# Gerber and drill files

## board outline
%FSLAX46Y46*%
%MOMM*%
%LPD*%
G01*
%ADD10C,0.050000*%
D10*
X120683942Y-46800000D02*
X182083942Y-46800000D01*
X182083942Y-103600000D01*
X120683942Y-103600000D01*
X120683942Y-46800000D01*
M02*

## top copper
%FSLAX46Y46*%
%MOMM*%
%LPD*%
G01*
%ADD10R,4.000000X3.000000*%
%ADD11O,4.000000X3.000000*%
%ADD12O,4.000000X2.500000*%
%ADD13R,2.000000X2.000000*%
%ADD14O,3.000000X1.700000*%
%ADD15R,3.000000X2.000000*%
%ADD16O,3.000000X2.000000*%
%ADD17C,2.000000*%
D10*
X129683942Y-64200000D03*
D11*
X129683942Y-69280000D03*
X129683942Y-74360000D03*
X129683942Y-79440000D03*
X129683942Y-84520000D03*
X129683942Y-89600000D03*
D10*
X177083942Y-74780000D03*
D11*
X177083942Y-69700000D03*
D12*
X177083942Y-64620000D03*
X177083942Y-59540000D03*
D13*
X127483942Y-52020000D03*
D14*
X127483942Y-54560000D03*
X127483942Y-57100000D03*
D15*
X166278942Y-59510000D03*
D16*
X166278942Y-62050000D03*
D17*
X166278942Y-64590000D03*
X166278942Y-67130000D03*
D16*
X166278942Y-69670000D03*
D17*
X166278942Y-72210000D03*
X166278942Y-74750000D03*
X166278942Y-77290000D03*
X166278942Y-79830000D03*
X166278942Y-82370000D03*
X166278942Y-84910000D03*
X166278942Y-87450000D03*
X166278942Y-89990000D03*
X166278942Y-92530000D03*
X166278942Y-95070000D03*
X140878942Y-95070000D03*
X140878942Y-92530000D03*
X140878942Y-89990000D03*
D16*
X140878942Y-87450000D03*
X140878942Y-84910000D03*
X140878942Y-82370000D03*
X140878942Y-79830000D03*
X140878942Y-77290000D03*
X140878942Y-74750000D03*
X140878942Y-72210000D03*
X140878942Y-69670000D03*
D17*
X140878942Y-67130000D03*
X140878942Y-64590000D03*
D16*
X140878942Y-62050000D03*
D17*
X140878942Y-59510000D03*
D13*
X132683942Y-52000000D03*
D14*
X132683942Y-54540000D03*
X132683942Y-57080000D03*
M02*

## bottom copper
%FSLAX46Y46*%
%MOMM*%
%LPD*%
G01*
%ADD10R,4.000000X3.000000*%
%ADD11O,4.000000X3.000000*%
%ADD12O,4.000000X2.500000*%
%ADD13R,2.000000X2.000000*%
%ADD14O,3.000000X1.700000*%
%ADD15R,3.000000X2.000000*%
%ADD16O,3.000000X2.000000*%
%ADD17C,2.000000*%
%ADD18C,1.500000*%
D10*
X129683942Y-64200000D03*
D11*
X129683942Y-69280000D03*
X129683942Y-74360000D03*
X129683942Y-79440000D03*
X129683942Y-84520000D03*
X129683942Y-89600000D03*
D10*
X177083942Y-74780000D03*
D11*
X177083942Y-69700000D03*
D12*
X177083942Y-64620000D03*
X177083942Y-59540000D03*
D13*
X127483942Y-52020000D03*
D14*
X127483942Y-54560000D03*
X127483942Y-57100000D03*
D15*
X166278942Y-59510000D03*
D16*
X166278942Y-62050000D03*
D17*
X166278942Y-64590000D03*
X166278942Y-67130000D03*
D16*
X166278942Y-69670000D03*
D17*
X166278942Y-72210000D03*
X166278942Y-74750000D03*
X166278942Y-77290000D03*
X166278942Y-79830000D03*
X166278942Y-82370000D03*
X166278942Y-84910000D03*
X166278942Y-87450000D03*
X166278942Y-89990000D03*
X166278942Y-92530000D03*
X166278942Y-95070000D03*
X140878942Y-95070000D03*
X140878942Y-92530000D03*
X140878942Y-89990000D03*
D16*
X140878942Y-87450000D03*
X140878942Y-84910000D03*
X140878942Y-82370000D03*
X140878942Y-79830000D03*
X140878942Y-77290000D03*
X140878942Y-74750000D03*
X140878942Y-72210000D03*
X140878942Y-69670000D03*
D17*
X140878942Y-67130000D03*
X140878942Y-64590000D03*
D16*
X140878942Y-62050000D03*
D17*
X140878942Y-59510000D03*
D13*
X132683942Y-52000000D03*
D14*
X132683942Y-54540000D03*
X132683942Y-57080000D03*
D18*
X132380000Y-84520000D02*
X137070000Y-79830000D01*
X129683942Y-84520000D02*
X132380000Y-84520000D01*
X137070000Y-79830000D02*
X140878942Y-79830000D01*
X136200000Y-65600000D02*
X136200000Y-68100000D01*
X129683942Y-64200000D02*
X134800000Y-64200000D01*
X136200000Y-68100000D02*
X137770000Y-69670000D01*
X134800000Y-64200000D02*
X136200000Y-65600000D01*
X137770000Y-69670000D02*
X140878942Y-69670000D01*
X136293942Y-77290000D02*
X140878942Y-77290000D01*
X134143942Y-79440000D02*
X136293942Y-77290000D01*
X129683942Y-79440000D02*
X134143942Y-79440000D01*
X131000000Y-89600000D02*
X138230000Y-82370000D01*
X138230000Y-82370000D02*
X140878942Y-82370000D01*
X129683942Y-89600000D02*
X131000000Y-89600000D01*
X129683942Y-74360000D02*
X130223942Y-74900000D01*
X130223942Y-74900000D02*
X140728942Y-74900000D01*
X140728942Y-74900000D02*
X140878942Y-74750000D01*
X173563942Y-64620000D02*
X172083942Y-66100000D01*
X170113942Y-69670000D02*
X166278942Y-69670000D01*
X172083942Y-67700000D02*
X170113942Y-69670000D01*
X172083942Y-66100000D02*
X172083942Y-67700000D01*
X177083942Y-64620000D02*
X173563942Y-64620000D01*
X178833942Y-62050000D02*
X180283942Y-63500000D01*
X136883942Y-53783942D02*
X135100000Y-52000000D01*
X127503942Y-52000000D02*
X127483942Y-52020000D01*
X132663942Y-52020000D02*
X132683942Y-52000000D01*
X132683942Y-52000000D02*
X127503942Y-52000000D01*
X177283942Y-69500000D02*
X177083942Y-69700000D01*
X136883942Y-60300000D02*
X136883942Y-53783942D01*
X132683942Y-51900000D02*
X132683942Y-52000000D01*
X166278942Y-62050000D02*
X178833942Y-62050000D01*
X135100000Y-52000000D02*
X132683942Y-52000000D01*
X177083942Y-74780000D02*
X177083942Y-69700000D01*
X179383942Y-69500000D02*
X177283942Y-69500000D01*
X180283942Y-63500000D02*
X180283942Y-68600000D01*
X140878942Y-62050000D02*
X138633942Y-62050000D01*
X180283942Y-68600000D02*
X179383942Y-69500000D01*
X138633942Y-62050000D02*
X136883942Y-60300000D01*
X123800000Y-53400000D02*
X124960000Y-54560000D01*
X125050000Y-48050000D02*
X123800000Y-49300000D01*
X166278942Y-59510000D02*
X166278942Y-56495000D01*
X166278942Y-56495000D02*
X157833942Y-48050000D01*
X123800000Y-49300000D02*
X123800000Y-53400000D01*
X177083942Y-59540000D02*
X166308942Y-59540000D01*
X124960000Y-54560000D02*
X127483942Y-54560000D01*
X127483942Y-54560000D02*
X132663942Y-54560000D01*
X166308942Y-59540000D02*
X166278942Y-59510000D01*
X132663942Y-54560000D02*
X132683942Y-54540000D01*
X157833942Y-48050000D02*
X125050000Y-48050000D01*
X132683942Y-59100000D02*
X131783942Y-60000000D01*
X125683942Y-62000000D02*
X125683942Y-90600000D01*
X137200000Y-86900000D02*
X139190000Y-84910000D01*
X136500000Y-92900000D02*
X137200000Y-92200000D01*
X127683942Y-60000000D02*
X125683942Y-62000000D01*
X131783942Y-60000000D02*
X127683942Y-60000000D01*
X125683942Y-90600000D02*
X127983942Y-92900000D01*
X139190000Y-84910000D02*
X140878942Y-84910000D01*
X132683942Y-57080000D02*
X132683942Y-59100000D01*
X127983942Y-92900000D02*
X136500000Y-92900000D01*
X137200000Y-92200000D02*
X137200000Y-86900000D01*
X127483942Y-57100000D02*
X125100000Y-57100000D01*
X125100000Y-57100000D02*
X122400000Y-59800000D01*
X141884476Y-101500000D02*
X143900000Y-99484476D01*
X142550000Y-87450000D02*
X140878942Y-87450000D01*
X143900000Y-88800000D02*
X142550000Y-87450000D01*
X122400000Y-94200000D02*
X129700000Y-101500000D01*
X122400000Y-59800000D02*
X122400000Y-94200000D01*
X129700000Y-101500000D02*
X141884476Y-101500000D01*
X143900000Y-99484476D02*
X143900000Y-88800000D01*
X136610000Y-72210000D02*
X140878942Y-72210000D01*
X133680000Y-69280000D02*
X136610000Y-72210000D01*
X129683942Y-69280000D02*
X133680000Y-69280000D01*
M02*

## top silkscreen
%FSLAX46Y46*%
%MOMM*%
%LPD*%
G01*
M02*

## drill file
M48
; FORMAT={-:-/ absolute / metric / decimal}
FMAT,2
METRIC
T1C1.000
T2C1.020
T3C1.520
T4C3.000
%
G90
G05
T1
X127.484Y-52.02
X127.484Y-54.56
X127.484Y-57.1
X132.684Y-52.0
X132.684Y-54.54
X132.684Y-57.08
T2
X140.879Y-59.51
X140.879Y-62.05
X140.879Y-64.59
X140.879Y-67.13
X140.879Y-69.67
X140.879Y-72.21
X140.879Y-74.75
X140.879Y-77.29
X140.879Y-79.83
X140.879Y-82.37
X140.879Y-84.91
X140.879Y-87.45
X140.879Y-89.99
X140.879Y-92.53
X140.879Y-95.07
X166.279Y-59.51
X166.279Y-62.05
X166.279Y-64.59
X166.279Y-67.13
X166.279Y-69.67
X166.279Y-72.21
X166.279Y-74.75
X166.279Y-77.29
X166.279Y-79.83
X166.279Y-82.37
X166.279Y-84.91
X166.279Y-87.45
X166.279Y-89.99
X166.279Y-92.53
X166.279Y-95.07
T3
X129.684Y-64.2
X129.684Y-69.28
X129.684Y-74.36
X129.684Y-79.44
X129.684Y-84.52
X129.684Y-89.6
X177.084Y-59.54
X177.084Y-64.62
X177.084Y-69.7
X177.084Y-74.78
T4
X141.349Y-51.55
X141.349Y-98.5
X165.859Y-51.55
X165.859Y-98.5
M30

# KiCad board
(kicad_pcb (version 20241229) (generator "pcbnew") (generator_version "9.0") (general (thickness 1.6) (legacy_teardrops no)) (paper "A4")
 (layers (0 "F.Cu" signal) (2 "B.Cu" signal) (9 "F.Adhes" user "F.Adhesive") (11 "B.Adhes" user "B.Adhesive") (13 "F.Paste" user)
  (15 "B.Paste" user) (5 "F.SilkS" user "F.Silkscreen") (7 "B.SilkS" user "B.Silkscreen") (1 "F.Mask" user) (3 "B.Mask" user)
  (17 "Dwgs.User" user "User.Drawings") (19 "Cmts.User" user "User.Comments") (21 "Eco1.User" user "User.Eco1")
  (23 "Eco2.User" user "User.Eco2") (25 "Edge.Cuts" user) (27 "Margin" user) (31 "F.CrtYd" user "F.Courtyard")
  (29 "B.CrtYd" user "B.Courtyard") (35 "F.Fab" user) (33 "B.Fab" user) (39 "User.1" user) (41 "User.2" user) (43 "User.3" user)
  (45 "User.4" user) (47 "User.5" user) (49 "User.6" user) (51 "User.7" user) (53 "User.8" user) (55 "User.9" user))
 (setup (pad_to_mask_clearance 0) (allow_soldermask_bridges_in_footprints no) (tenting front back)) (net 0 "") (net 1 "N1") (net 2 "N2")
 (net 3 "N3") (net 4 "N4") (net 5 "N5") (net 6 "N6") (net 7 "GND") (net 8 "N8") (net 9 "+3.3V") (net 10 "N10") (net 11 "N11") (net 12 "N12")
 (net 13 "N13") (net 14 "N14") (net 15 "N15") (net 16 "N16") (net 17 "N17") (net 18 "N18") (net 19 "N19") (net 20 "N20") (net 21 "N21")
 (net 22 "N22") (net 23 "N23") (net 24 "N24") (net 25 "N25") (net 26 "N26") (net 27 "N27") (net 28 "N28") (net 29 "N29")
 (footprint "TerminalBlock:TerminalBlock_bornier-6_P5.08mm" (layer "B.Cu") (at 129.683942 64.2 -90)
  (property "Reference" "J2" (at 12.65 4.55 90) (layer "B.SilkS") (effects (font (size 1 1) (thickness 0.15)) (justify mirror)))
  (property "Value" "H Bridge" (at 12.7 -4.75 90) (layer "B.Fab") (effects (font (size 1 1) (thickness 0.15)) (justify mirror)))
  (pad "1" thru_hole rect (at 0 0 270) (size 3 4) (drill 1.52) (layers "*.Cu" "*.Mask") (remove_unused_layers no) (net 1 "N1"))
  (pad "2" thru_hole oval (at 5.08 0 270) (size 3 4) (drill 1.52) (layers "*.Cu" "*.Mask") (remove_unused_layers no) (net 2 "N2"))
  (pad "3" thru_hole oval (at 10.16 0 270) (size 3 4) (drill 1.52) (layers "*.Cu" "*.Mask") (remove_unused_layers no) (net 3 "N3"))
  (pad "4" thru_hole oval (at 15.24 0 270) (size 3 4) (drill 1.52) (layers "*.Cu" "*.Mask") (remove_unused_layers no) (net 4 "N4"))
  (pad "5" thru_hole oval (at 20.32 0 270) (size 3 4) (drill 1.52) (layers "*.Cu" "*.Mask") (remove_unused_layers no) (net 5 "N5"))
  (pad "6" thru_hole oval (at 25.4 0 270) (size 3 4) (drill 1.52) (layers "*.Cu" "*.Mask") (remove_unused_layers no) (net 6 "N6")))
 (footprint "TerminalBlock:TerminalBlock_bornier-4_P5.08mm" (layer "B.Cu") (at 177.083942 74.78 90)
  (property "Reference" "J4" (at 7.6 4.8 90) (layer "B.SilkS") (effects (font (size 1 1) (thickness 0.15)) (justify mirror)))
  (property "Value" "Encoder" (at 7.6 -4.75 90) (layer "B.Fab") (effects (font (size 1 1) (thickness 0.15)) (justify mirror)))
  (pad "1" thru_hole rect (at 0 0 90) (size 3 4) (drill 1.52) (layers "*.Cu" "*.Mask") (remove_unused_layers no) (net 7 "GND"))
  (pad "2" thru_hole oval (at 5.08 0 90) (size 3 4) (drill 1.52) (layers "*.Cu" "*.Mask") (remove_unused_layers no) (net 7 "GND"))
  (pad "3" thru_hole oval (at 10.16 0 90) (size 2.5 4) (drill 1.52) (layers "*.Cu" "*.Mask") (remove_unused_layers no) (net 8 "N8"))
  (pad "4" thru_hole oval (at 15.24 0 90) (size 2.5 4) (drill 1.52) (layers "*.Cu" "*.Mask") (remove_unused_layers no) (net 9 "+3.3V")))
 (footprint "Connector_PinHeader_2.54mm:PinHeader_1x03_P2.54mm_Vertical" (layer "B.Cu") (at 127.483942 52.02 180)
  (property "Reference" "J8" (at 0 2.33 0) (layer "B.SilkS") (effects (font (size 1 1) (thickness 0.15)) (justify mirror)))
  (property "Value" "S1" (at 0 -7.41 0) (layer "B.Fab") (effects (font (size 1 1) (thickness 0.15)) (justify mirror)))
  (pad "1" thru_hole rect (at 0 0 180) (size 2 2) (drill 1) (layers "*.Cu" "*.Mask") (remove_unused_layers no) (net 7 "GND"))
  (pad "2" thru_hole oval (at 0 -2.54 180) (size 3 1.7) (drill 1) (layers "*.Cu" "*.Mask") (remove_unused_layers no) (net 9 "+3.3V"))
  (pad "3" thru_hole oval (at 0 -5.08 180) (size 3 1.7) (drill 1) (layers "*.Cu" "*.Mask") (remove_unused_layers no) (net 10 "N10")))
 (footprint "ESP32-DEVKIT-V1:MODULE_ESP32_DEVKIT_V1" (layer "B.Cu") (at 153.578942 75.025 180)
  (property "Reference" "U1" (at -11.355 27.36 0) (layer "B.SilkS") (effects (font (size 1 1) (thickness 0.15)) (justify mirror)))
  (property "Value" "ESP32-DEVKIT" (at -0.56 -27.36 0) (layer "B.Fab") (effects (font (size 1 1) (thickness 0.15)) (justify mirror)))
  (pad "" np_thru_hole circle (at -12.28 -23.475 180) (size 3 3) (drill 3) (layers "*.Cu" "*.Mask"))
  (pad "" np_thru_hole circle (at -12.28 23.475 180) (size 3 3) (drill 3) (layers "*.Cu" "*.Mask"))
  (pad "" np_thru_hole circle (at 12.23 -23.475 180) (size 3 3) (drill 3) (layers "*.Cu" "*.Mask"))
  (pad "" np_thru_hole circle (at 12.23 23.475 180) (size 3 3) (drill 3) (layers "*.Cu" "*.Mask"))
  (pad "1" thru_hole rect (at -12.7 15.515 180) (size 3 2) (drill 1.02) (layers "*.Cu" "*.Mask") (remove_unused_layers no) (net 9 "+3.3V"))
  (pad "2" thru_hole oval (at -12.7 12.975 180) (size 3 2) (drill 1.02) (layers "*.Cu" "*.Mask") (remove_unused_layers no) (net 7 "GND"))
  (pad "3" thru_hole circle (at -12.7 10.435 180) (size 2 2) (drill 1.02) (layers "*.Cu" "*.Mask") (remove_unused_layers no) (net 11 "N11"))
  (pad "4" thru_hole circle (at -12.7 7.895 180) (size 2 2) (drill 1.02) (layers "*.Cu" "*.Mask") (remove_unused_layers no) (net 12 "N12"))
  (pad "5" thru_hole oval (at -12.7 5.355 180) (size 3 2) (drill 1.02) (layers "*.Cu" "*.Mask") (remove_unused_layers no) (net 8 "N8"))
  (pad "6" thru_hole circle (at -12.7 2.815 180) (size 2 2) (drill 1.02) (layers "*.Cu" "*.Mask") (remove_unused_layers no) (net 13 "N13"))
  (pad "7" thru_hole circle (at -12.7 0.275 180) (size 2 2) (drill 1.02) (layers "*.Cu" "*.Mask") (remove_unused_layers no) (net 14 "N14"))
  (pad "8" thru_hole circle (at -12.7 -2.265 180) (size 2 2) (drill 1.02) (layers "*.Cu" "*.Mask") (remove_unused_layers no) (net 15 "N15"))
  (pad "9" thru_hole circle (at -12.7 -4.805 180) (size 2 2) (drill 1.02) (layers "*.Cu" "*.Mask") (remove_unused_layers no) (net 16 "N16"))
  (pad "10" thru_hole circle (at -12.7 -7.345 180) (size 2 2) (drill 1.02) (layers "*.Cu" "*.Mask") (remove_unused_layers no) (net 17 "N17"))
  (pad "11" thru_hole circle (at -12.7 -9.885 180) (size 2 2) (drill 1.02) (layers "*.Cu" "*.Mask") (remove_unused_layers no) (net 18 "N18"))
  (pad "12" thru_hole circle (at -12.7 -12.425 180) (size 2 2) (drill 1.02) (layers "*.Cu" "*.Mask") (remove_unused_layers no)
   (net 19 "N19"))
  (pad "13" thru_hole circle (at -12.7 -14.965 180) (size 2 2) (drill 1.02) (layers "*.Cu" "*.Mask") (remove_unused_layers no)
   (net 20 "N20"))
  (pad "14" thru_hole circle (at -12.7 -17.505 180) (size 2 2) (drill 1.02) (layers "*.Cu" "*.Mask") (remove_unused_layers no)
   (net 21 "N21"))
  (pad "15" thru_hole circle (at -12.7 -20.045 180) (size 2 2) (drill 1.02) (layers "*.Cu" "*.Mask") (remove_unused_layers no)
   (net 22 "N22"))
  (pad "16" thru_hole circle (at 12.7 -20.045 180) (size 2 2) (drill 1.02) (layers "*.Cu" "*.Mask") (remove_unused_layers no) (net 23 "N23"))
  (pad "17" thru_hole circle (at 12.7 -17.505 180) (size 2 2) (drill 1.02) (layers "*.Cu" "*.Mask") (remove_unused_layers no) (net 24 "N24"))
  (pad "18" thru_hole circle (at 12.7 -14.965 180) (size 2 2) (drill 1.02) (layers "*.Cu" "*.Mask") (remove_unused_layers no) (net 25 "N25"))
  (pad "19" thru_hole oval (at 12.7 -12.425 180) (size 3 2) (drill 1.02) (layers "*.Cu" "*.Mask") (remove_unused_layers no) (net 10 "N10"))
  (pad "20" thru_hole oval (at 12.7 -9.885 180) (size 3 2) (drill 1.02) (layers "*.Cu" "*.Mask") (remove_unused_layers no) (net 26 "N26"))
  (pad "21" thru_hole oval (at 12.7 -7.345 180) (size 3 2) (drill 1.02) (layers "*.Cu" "*.Mask") (remove_unused_layers no) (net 6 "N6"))
  (pad "22" thru_hole oval (at 12.7 -4.805 180) (size 3 2) (drill 1.02) (layers "*.Cu" "*.Mask") (remove_unused_layers no) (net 5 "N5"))
  (pad "23" thru_hole oval (at 12.7 -2.265 180) (size 3 2) (drill 1.02) (layers "*.Cu" "*.Mask") (remove_unused_layers no) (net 4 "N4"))
  (pad "24" thru_hole oval (at 12.7 0.275 180) (size 3 2) (drill 1.02) (layers "*.Cu" "*.Mask") (remove_unused_layers no) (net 3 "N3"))
  (pad "25" thru_hole oval (at 12.7 2.815 180) (size 3 2) (drill 1.02) (layers "*.Cu" "*.Mask") (remove_unused_layers no) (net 2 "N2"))
  (pad "26" thru_hole oval (at 12.7 5.355 180) (size 3 2) (drill 1.02) (layers "*.Cu" "*.Mask") (remove_unused_layers no) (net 1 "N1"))
  (pad "27" thru_hole circle (at 12.7 7.895 180) (size 2 2) (drill 1.02) (layers "*.Cu" "*.Mask") (remove_unused_layers no) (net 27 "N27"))
  (pad "28" thru_hole circle (at 12.7 10.435 180) (size 2 2) (drill 1.02) (layers "*.Cu" "*.Mask") (remove_unused_layers no) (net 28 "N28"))
  (pad "29" thru_hole oval (at 12.7 12.975 180) (size 3 2) (drill 1.02) (layers "*.Cu" "*.Mask") (remove_unused_layers no) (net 7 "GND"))
  (pad "30" thru_hole circle (at 12.7 15.515 180) (size 2 2) (drill 1.02) (layers "*.Cu" "*.Mask") (remove_unused_layers no) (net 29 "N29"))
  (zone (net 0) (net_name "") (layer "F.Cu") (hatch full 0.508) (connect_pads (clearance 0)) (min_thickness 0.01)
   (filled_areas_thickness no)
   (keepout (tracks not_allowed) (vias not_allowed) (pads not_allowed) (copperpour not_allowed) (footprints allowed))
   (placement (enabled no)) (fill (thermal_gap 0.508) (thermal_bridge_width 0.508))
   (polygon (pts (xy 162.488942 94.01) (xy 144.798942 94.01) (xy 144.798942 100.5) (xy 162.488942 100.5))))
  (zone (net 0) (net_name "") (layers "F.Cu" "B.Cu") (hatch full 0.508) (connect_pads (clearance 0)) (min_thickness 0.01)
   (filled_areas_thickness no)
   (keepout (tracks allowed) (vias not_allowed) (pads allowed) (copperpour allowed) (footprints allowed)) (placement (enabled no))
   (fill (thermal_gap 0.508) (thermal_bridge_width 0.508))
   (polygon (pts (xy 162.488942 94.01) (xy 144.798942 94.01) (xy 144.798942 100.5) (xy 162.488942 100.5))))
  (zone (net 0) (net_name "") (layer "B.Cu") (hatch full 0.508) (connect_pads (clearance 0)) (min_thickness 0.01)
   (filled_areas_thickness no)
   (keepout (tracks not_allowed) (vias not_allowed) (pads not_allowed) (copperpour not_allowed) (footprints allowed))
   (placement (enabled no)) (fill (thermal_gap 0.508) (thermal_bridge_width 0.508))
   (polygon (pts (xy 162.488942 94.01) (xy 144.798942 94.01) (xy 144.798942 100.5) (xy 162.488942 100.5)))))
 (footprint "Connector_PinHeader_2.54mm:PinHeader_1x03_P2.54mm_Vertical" (layer "B.Cu") (at 132.683942 52 180)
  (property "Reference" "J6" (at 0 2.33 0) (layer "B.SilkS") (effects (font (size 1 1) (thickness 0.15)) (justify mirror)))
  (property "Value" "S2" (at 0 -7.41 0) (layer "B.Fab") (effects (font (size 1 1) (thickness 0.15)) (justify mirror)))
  (pad "1" thru_hole rect (at 0 0 180) (size 2 2) (drill 1) (layers "*.Cu" "*.Mask") (remove_unused_layers no) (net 7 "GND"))
  (pad "2" thru_hole oval (at 0 -2.54 180) (size 3 1.7) (drill 1) (layers "*.Cu" "*.Mask") (remove_unused_layers no) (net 9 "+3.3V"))
  (pad "3" thru_hole oval (at 0 -5.08 180) (size 3 1.7) (drill 1) (layers "*.Cu" "*.Mask") (remove_unused_layers no) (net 26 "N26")))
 (gr_rect (start 120.683942 46.8) (end 182.083942 103.6) (stroke (width 0.05) (type default)) (fill no) (layer "Edge.Cuts"))
 (segment (start 132.38 84.52) (end 137.07 79.83) (width 1.5) (layer "B.Cu") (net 5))
 (segment (start 129.683942 84.52) (end 132.38 84.52) (width 1.5) (layer "B.Cu") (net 5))
 (segment (start 137.07 79.83) (end 140.878942 79.83) (width 1.5) (layer "B.Cu") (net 5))
 (segment (start 136.2 65.6) (end 136.2 68.1) (width 1.5) (layer "B.Cu") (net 1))
 (segment (start 129.683942 64.2) (end 134.8 64.2) (width 1.5) (layer "B.Cu") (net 1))
 (segment (start 136.2 68.1) (end 137.77 69.67) (width 1.5) (layer "B.Cu") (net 1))
 (segment (start 134.8 64.2) (end 136.2 65.6) (width 1.5) (layer "B.Cu") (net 1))
 (segment (start 137.77 69.67) (end 140.878942 69.67) (width 1.5) (layer "B.Cu") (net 1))
 (segment (start 136.293942 77.29) (end 140.878942 77.29) (width 1.5) (layer "B.Cu") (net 4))
 (segment (start 134.143942 79.44) (end 136.293942 77.29) (width 1.5) (layer "B.Cu") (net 4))
 (segment (start 129.683942 79.44) (end 134.143942 79.44) (width 1.5) (layer "B.Cu") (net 4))
 (segment (start 131 89.6) (end 138.23 82.37) (width 1.5) (layer "B.Cu") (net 6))
 (segment (start 138.23 82.37) (end 140.878942 82.37) (width 1.5) (layer "B.Cu") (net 6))
 (segment (start 129.683942 89.6) (end 131 89.6) (width 1.5) (layer "B.Cu") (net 6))
 (segment (start 129.683942 74.36) (end 130.223942 74.9) (width 1.5) (layer "B.Cu") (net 3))
 (segment (start 130.223942 74.9) (end 140.728942 74.9) (width 1.5) (layer "B.Cu") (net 3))
 (segment (start 140.728942 74.9) (end 140.878942 74.75) (width 1.5) (layer "B.Cu") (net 3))
 (segment (start 173.563942 64.62) (end 172.083942 66.1) (width 1.5) (layer "B.Cu") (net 8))
 (segment (start 170.113942 69.67) (end 166.278942 69.67) (width 1.5) (layer "B.Cu") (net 8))
 (segment (start 172.083942 67.7) (end 170.113942 69.67) (width 1.5) (layer "B.Cu") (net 8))
 (segment (start 172.083942 66.1) (end 172.083942 67.7) (width 1.5) (layer "B.Cu") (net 8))
 (segment (start 177.083942 64.62) (end 173.563942 64.62) (width 1.5) (layer "B.Cu") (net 8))
 (segment (start 178.833942 62.05) (end 180.283942 63.5) (width 1.5) (layer "B.Cu") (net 7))
 (segment (start 136.883942 53.783942) (end 135.1 52) (width 1.5) (layer "B.Cu") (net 7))
 (segment (start 127.503942 52) (end 127.483942 52.02) (width 1.5) (layer "B.Cu") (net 7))
 (segment (start 132.663942 52.02) (end 132.683942 52) (width 1.5) (layer "B.Cu") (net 7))
 (segment (start 132.683942 52) (end 127.503942 52) (width 1.5) (layer "B.Cu") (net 7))
 (segment (start 177.283942 69.5) (end 177.083942 69.7) (width 1.5) (layer "B.Cu") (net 7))
 (segment (start 136.883942 60.3) (end 136.883942 53.783942) (width 1.5) (layer "B.Cu") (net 7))
 (segment (start 132.683942 51.9) (end 132.683942 52) (width 1.5) (layer "B.Cu") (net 7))
 (segment (start 166.278942 62.05) (end 178.833942 62.05) (width 1.5) (layer "B.Cu") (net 7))
 (segment (start 135.1 52) (end 132.683942 52) (width 1.5) (layer "B.Cu") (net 7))
 (segment (start 177.083942 74.78) (end 177.083942 69.7) (width 1.5) (layer "B.Cu") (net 7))
 (segment (start 179.383942 69.5) (end 177.283942 69.5) (width 1.5) (layer "B.Cu") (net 7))
 (segment (start 180.283942 63.5) (end 180.283942 68.6) (width 1.5) (layer "B.Cu") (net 7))
 (segment (start 140.878942 62.05) (end 138.633942 62.05) (width 1.5) (layer "B.Cu") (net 7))
 (segment (start 180.283942 68.6) (end 179.383942 69.5) (width 1.5) (layer "B.Cu") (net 7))
 (segment (start 138.633942 62.05) (end 136.883942 60.3) (width 1.5) (layer "B.Cu") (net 7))
 (segment (start 123.8 53.4) (end 124.96 54.56) (width 1.5) (layer "B.Cu") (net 9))
 (segment (start 125.05 48.05) (end 123.8 49.3) (width 1.5) (layer "B.Cu") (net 9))
 (segment (start 166.278942 59.51) (end 166.278942 56.495) (width 1.5) (layer "B.Cu") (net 9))
 (segment (start 166.278942 56.495) (end 157.833942 48.05) (width 1.5) (layer "B.Cu") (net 9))
 (segment (start 123.8 49.3) (end 123.8 53.4) (width 1.5) (layer "B.Cu") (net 9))
 (segment (start 177.083942 59.54) (end 166.308942 59.54) (width 1.5) (layer "B.Cu") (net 9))
 (segment (start 124.96 54.56) (end 127.483942 54.56) (width 1.5) (layer "B.Cu") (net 9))
 (segment (start 127.483942 54.56) (end 132.663942 54.56) (width 1.5) (layer "B.Cu") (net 9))
 (segment (start 166.308942 59.54) (end 166.278942 59.51) (width 1.5) (layer "B.Cu") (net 9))
 (segment (start 132.663942 54.56) (end 132.683942 54.54) (width 1.5) (layer "B.Cu") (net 9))
 (segment (start 157.833942 48.05) (end 125.05 48.05) (width 1.5) (layer "B.Cu") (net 9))
 (segment (start 132.683942 59.1) (end 131.783942 60) (width 1.5) (layer "B.Cu") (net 26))
 (segment (start 125.683942 62) (end 125.683942 90.6) (width 1.5) (layer "B.Cu") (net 26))
 (segment (start 137.2 86.9) (end 139.19 84.91) (width 1.5) (layer "B.Cu") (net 26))
 (segment (start 136.5 92.9) (end 137.2 92.2) (width 1.5) (layer "B.Cu") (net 26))
 (segment (start 127.683942 60) (end 125.683942 62) (width 1.5) (layer "B.Cu") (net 26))
 (segment (start 131.783942 60) (end 127.683942 60) (width 1.5) (layer "B.Cu") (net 26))
 (segment (start 125.683942 90.6) (end 127.983942 92.9) (width 1.5) (layer "B.Cu") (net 26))
 (segment (start 139.19 84.91) (end 140.878942 84.91) (width 1.5) (layer "B.Cu") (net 26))
 (segment (start 132.683942 57.08) (end 132.683942 59.1) (width 1.5) (layer "B.Cu") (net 26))
 (segment (start 127.983942 92.9) (end 136.5 92.9) (width 1.5) (layer "B.Cu") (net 26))
 (segment (start 137.2 92.2) (end 137.2 86.9) (width 1.5) (layer "B.Cu") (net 26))
 (segment (start 127.483942 57.1) (end 125.1 57.1) (width 1.5) (layer "B.Cu") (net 10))
 (segment (start 125.1 57.1) (end 122.4 59.8) (width 1.5) (layer "B.Cu") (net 10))
 (segment (start 141.884476 101.5) (end 143.9 99.484476) (width 1.5) (layer "B.Cu") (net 10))
 (segment (start 142.55 87.45) (end 140.878942 87.45) (width 1.5) (layer "B.Cu") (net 10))
 (segment (start 143.9 88.8) (end 142.55 87.45) (width 1.5) (layer "B.Cu") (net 10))
 (segment (start 122.4 94.2) (end 129.7 101.5) (width 1.5) (layer "B.Cu") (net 10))
 (segment (start 122.4 59.8) (end 122.4 94.2) (width 1.5) (layer "B.Cu") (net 10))
 (segment (start 129.7 101.5) (end 141.884476 101.5) (width 1.5) (layer "B.Cu") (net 10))
 (segment (start 143.9 99.484476) (end 143.9 88.8) (width 1.5) (layer "B.Cu") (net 10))
 (segment (start 136.61 72.21) (end 140.878942 72.21) (width 1.5) (layer "B.Cu") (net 2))
 (segment (start 133.68 69.28) (end 136.61 72.21) (width 1.5) (layer "B.Cu") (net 2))
 (segment (start 129.683942 69.28) (end 133.68 69.28) (width 1.5) (layer "B.Cu") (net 2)))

